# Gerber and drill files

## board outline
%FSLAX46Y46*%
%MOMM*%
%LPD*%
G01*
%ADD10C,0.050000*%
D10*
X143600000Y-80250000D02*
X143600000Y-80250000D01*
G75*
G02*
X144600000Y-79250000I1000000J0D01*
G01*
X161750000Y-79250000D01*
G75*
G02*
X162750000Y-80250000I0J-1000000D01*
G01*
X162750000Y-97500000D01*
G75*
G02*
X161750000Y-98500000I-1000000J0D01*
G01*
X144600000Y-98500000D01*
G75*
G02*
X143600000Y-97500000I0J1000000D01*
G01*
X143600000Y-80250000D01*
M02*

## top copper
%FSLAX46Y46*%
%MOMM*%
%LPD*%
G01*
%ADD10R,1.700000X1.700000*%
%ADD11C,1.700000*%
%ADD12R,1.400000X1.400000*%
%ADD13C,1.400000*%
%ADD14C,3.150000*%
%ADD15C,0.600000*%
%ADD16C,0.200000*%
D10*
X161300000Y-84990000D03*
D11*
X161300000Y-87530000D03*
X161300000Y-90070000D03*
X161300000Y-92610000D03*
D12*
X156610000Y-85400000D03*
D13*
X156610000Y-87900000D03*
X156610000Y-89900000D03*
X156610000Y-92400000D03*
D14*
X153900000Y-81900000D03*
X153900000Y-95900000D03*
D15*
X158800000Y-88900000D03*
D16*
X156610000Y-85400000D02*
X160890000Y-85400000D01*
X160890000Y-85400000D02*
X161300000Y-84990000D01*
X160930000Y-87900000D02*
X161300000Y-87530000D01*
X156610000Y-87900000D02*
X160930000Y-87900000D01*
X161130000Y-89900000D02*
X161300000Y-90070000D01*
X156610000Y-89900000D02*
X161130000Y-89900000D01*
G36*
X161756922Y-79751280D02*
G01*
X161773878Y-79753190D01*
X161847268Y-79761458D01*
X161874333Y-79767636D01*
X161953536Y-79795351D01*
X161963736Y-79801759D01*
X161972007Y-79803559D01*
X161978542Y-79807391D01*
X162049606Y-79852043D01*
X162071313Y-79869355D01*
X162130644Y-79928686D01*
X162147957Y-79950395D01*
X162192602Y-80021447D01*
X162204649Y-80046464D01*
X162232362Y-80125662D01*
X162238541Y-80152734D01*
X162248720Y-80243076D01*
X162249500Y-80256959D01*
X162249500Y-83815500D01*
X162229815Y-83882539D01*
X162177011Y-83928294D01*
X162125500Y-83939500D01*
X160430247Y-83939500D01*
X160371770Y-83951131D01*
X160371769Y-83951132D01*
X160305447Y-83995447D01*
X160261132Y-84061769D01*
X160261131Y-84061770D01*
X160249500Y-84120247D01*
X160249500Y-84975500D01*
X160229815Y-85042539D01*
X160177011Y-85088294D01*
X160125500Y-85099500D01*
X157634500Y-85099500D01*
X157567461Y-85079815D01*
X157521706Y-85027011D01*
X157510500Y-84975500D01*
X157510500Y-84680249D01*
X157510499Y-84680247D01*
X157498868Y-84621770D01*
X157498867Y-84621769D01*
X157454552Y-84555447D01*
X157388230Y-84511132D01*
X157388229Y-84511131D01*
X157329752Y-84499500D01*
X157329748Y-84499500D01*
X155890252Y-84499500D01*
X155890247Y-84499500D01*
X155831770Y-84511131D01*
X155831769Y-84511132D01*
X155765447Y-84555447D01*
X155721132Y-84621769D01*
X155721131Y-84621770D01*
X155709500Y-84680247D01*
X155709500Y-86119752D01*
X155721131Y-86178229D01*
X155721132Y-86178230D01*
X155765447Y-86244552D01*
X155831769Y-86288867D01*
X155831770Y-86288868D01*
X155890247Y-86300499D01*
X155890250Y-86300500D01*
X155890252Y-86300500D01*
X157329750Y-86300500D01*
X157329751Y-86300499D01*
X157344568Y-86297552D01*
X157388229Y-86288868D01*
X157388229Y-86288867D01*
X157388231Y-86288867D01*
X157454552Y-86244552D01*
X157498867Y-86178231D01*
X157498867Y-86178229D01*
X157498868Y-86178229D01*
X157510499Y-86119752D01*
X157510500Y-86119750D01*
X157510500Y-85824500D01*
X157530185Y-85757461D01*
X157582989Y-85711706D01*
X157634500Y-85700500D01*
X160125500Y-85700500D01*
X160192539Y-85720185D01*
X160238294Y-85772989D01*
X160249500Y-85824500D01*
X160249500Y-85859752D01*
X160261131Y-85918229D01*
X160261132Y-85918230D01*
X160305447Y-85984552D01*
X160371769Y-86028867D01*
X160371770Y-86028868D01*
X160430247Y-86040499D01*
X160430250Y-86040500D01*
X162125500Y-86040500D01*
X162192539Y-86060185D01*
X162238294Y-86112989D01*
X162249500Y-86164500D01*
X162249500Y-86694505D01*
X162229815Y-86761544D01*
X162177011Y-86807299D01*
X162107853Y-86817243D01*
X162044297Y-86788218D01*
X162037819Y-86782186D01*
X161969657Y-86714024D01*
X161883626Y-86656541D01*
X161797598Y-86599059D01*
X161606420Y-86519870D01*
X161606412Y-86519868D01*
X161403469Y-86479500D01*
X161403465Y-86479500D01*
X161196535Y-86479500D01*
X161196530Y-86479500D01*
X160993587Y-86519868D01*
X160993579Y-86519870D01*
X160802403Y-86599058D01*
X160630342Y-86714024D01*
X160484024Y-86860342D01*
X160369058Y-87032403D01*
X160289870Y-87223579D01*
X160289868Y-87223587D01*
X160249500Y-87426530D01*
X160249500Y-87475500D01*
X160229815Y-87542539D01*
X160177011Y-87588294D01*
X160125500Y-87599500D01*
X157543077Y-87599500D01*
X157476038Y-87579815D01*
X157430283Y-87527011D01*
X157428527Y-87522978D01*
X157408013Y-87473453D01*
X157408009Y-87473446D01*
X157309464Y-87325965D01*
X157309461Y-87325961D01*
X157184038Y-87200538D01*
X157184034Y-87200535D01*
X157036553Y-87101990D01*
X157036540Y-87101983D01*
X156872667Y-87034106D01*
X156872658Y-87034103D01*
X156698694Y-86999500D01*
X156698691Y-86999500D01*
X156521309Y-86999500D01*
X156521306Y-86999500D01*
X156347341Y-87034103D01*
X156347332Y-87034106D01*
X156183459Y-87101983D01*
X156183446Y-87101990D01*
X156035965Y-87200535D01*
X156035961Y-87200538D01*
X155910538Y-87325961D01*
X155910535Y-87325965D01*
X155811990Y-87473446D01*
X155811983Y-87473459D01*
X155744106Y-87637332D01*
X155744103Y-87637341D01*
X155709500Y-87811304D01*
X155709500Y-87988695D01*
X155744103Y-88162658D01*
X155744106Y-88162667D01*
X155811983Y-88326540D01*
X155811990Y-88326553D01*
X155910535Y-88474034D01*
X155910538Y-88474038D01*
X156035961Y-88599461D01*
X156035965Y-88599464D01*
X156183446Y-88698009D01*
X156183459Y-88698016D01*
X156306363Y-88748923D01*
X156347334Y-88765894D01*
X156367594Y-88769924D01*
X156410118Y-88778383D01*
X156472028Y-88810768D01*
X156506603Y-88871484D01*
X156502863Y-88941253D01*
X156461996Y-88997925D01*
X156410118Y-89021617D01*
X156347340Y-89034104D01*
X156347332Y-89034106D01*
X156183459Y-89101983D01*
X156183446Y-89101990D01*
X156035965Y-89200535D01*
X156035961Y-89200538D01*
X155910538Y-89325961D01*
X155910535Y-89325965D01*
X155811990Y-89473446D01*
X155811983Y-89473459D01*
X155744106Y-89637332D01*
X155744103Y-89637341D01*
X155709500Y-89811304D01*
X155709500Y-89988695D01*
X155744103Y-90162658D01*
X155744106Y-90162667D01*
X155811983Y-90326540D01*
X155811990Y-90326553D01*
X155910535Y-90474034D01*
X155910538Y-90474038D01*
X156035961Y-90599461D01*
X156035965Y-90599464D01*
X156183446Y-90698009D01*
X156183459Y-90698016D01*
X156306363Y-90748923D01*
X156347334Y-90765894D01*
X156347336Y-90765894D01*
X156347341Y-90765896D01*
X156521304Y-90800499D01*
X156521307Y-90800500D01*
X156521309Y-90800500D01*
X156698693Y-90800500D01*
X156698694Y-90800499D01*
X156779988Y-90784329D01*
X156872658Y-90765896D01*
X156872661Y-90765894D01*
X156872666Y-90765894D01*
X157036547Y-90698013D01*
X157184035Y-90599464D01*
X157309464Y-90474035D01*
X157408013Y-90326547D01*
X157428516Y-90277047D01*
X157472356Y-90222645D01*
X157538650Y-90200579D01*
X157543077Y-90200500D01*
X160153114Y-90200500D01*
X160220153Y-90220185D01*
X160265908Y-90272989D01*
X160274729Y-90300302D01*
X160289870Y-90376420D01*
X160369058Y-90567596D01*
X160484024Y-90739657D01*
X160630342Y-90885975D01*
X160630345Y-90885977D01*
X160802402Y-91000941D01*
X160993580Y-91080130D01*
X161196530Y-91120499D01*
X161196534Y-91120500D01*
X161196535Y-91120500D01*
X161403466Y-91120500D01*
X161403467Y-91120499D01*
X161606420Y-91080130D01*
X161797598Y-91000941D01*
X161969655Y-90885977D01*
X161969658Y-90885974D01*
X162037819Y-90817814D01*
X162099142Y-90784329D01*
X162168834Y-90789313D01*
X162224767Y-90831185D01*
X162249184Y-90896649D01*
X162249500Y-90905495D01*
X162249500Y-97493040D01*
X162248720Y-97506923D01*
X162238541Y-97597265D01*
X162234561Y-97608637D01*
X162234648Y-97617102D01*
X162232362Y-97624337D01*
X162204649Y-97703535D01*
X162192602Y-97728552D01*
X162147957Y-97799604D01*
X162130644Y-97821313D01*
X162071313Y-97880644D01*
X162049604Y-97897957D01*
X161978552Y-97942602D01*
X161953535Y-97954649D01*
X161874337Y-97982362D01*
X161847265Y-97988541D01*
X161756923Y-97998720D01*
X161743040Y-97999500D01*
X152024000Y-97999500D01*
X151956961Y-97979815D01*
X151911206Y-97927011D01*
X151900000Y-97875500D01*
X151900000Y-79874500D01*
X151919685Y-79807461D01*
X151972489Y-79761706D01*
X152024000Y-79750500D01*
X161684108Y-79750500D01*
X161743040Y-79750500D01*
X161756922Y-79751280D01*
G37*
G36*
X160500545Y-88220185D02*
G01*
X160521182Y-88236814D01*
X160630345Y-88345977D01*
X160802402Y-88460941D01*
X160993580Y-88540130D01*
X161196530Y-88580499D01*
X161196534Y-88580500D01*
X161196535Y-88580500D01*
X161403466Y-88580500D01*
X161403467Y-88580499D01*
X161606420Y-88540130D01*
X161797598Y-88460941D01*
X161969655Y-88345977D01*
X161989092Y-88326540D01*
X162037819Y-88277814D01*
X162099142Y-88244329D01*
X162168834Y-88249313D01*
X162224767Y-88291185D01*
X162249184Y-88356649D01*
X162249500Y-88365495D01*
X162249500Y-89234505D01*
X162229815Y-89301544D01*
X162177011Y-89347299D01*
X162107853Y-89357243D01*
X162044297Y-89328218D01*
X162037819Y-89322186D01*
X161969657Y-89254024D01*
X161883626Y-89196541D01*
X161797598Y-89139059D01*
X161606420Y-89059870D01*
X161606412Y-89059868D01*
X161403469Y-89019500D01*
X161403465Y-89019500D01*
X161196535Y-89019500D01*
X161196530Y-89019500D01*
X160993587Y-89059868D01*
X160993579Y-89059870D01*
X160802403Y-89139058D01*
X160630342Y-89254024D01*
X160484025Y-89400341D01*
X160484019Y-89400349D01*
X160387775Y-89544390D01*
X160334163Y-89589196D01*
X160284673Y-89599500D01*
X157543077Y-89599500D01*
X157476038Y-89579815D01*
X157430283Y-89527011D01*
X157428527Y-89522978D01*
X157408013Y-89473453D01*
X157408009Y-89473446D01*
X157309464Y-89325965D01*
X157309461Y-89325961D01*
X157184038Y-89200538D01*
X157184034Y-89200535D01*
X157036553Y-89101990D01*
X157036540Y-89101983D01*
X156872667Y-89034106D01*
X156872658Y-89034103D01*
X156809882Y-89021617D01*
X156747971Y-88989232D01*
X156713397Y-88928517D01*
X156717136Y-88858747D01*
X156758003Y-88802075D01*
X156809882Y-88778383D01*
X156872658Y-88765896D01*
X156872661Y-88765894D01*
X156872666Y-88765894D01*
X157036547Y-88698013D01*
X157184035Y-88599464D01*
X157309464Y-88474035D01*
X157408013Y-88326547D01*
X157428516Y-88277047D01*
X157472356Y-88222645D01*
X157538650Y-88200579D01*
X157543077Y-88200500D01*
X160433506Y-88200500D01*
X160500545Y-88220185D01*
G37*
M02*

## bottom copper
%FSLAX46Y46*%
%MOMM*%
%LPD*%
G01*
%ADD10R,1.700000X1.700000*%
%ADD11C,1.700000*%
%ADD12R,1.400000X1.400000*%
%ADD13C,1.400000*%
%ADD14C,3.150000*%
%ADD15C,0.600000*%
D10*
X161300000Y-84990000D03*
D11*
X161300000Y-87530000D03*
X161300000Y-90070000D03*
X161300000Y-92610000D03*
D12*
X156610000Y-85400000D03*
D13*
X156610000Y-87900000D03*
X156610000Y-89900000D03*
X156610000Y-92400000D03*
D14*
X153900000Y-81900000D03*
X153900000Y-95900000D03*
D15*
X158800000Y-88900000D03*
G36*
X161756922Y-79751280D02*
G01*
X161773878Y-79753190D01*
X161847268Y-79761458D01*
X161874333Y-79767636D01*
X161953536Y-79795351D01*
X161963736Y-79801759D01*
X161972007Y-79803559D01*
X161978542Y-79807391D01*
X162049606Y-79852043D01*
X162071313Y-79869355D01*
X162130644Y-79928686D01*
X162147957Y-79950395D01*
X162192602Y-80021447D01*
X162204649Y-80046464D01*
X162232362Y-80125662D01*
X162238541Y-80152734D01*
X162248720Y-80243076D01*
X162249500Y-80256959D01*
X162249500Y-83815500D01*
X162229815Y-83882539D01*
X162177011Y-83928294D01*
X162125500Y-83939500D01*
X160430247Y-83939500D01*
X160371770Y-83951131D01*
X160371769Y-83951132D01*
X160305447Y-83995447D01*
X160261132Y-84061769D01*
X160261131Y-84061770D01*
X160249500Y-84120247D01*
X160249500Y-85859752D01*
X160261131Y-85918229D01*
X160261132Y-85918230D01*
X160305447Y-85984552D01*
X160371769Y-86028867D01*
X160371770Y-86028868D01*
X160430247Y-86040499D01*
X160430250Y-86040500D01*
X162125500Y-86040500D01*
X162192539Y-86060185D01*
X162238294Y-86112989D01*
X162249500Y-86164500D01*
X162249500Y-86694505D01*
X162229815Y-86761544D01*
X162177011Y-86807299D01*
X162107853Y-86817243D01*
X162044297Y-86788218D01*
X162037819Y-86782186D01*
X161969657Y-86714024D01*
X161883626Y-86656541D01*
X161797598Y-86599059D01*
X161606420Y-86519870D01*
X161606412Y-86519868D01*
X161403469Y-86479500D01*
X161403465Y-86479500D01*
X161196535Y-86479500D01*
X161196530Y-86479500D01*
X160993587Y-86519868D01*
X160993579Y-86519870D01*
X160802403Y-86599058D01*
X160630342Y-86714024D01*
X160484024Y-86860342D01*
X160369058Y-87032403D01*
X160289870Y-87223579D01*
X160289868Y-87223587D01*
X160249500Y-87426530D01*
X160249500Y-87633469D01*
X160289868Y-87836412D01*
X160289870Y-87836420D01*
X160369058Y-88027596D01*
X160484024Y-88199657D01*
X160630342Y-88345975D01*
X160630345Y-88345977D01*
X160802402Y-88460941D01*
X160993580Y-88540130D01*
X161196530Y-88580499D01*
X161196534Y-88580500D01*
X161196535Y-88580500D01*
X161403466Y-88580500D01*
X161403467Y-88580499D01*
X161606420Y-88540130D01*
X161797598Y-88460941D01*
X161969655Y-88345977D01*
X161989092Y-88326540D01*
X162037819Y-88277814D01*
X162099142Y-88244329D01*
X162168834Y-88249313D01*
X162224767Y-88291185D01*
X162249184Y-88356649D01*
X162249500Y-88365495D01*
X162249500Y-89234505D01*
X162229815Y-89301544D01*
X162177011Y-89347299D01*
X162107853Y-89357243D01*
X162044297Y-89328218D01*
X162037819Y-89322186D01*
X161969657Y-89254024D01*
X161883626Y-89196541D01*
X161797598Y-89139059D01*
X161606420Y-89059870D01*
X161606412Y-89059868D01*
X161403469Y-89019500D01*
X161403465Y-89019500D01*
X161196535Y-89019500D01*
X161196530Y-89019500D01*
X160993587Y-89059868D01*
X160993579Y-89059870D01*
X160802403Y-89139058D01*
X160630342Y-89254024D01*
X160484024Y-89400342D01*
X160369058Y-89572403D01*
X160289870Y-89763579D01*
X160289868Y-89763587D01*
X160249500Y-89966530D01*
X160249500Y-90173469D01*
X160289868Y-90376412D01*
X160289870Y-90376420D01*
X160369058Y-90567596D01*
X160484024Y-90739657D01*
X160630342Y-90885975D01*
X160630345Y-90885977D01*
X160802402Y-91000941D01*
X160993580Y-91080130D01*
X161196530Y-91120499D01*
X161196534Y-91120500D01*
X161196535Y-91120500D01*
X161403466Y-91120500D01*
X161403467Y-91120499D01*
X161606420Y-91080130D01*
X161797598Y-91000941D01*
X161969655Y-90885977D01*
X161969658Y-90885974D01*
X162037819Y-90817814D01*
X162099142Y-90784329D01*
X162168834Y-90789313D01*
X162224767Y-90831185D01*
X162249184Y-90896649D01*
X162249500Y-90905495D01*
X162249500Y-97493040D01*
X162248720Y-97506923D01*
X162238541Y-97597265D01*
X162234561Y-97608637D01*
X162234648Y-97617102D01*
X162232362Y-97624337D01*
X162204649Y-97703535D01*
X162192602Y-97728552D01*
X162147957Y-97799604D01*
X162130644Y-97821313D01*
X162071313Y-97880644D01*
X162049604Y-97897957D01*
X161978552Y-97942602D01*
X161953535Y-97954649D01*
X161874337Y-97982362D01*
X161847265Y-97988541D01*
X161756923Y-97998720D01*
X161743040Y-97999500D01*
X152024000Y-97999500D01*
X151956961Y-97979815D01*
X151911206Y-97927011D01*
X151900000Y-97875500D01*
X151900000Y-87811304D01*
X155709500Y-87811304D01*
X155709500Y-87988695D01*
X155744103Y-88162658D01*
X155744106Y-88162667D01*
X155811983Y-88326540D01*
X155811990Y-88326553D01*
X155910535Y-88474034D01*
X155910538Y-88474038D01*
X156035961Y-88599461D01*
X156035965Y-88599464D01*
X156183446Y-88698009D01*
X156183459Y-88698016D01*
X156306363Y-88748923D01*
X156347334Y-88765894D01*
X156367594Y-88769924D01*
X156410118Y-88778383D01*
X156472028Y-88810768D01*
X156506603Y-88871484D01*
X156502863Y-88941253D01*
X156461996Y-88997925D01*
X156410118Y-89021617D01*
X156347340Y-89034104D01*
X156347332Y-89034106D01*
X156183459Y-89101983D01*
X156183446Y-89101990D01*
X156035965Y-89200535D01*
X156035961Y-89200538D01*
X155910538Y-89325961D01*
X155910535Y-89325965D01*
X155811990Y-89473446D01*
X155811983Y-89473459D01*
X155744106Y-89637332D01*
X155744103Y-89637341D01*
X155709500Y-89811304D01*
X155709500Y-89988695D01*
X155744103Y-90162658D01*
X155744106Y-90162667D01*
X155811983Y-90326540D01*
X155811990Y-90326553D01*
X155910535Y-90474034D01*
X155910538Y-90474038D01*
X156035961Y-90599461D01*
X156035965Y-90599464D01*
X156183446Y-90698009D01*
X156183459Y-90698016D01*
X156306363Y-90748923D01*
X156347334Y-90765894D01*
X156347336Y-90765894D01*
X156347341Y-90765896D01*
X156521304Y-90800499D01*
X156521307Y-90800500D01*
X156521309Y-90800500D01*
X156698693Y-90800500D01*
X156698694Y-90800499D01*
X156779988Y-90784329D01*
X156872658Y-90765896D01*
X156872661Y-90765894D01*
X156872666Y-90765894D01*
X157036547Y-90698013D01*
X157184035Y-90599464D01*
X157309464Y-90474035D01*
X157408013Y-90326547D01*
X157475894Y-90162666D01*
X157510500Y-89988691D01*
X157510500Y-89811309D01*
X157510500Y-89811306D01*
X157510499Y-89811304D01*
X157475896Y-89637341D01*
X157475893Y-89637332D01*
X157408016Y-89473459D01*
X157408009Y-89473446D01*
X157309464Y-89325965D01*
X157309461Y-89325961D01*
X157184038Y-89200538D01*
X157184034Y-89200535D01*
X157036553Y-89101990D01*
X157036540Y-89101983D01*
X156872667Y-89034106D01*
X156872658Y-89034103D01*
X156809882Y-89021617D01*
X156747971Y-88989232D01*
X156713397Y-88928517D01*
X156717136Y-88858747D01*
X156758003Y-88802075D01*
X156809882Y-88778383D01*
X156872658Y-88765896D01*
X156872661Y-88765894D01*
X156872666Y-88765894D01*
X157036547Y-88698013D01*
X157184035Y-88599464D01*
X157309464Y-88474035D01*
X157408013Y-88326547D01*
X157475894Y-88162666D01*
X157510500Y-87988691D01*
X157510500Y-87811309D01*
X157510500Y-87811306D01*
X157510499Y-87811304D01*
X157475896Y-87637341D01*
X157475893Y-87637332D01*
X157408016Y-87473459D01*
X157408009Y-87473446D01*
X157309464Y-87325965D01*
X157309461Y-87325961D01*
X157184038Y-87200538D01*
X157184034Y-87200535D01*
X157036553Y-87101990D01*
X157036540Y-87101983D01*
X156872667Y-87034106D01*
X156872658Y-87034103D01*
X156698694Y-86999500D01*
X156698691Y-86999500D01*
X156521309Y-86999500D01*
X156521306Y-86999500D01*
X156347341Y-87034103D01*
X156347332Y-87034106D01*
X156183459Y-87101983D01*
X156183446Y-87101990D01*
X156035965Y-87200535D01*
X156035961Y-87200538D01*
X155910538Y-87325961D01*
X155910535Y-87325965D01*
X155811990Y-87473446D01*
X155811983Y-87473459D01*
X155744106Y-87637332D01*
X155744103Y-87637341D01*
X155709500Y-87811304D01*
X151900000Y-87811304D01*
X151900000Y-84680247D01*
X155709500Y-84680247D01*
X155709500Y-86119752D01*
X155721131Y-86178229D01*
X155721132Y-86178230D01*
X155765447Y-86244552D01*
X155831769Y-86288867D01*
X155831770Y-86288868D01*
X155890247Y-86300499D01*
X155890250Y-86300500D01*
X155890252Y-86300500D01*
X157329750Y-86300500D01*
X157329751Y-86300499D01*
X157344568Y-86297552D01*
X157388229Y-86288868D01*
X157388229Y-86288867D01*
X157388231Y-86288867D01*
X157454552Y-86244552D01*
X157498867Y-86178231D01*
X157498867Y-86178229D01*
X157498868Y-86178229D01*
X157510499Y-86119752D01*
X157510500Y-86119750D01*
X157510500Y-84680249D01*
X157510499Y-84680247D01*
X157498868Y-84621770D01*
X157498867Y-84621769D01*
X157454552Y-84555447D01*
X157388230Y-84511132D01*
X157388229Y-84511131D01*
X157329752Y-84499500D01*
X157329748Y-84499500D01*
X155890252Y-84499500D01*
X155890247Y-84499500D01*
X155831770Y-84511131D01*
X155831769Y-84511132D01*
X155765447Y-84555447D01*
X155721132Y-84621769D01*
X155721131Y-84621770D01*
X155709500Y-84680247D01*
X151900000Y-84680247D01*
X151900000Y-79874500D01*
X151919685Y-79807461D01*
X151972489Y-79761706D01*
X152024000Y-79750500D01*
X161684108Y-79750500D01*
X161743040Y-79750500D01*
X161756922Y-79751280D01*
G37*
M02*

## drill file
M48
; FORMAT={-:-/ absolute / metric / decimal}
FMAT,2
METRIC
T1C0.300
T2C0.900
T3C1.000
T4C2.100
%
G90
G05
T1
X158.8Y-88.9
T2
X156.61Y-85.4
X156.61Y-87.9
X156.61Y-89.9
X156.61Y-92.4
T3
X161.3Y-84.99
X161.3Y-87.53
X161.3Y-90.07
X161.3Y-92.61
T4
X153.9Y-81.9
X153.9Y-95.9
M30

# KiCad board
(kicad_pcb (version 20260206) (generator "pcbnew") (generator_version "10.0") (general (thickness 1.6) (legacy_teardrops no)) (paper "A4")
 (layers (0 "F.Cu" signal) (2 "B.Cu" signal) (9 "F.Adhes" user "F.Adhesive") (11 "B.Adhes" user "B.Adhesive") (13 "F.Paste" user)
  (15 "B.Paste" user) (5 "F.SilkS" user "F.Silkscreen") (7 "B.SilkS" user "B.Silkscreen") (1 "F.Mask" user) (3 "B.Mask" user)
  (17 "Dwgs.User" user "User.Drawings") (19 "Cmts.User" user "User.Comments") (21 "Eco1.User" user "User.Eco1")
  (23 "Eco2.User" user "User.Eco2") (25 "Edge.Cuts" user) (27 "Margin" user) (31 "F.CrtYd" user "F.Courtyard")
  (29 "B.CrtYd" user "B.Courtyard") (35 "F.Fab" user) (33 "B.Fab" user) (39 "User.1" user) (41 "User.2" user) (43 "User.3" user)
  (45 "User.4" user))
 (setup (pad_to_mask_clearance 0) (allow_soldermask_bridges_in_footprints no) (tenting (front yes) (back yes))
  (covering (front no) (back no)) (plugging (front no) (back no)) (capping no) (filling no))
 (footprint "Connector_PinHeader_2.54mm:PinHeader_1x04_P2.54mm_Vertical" (layer "F.Cu") (at 161.3 84.99)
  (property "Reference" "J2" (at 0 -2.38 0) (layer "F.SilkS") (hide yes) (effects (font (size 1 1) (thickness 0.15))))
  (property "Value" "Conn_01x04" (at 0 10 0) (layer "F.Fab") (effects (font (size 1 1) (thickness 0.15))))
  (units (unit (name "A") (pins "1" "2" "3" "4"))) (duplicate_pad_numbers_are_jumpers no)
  (pad "1" thru_hole rect (at 0 0) (size 1.7 1.7) (drill 1) (layers "*.Cu" "*.Mask") (remove_unused_layers no) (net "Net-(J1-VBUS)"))
  (pad "2" thru_hole circle (at 0 2.54) (size 1.7 1.7) (drill 1) (layers "*.Cu" "*.Mask") (remove_unused_layers no) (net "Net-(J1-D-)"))
  (pad "3" thru_hole circle (at 0 5.08) (size 1.7 1.7) (drill 1) (layers "*.Cu" "*.Mask") (remove_unused_layers no) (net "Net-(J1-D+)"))
  (pad "4" thru_hole circle (at 0 7.62) (size 1.7 1.7) (drill 1) (layers "*.Cu" "*.Mask") (remove_unused_layers no) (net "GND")))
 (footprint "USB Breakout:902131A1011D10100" (layer "F.Cu") (at 156.61 85.4 -90)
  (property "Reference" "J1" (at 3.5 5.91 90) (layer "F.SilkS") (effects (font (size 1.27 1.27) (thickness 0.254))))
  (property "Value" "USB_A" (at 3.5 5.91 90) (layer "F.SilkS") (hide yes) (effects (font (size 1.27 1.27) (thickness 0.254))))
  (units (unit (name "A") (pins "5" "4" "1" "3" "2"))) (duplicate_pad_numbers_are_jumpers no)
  (pad "1" thru_hole rect (at 0 0 270) (size 1.4 1.4) (drill 0.9) (layers "*.Cu" "*.Mask") (remove_unused_layers no) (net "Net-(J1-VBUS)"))
  (pad "2" thru_hole circle (at 2.5 0 270) (size 1.4 1.4) (drill 0.9) (layers "*.Cu" "*.Mask") (remove_unused_layers no) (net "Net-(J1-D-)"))
  (pad "3" thru_hole circle (at 4.5 0 270) (size 1.4 1.4) (drill 0.9) (layers "*.Cu" "*.Mask") (remove_unused_layers no) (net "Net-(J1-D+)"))
  (pad "4" thru_hole circle (at 7 0 270) (size 1.4 1.4) (drill 0.9) (layers "*.Cu" "*.Mask") (remove_unused_layers no) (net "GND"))
  (pad "5" thru_hole circle (at -3.5 2.71 270) (size 3.15 3.15) (drill 2.1) (layers "*.Cu" "*.Mask") (remove_unused_layers no) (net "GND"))
  (pad "5" thru_hole circle (at 10.5 2.71 270) (size 3.15 3.15) (drill 2.1) (layers "*.Cu" "*.Mask") (remove_unused_layers no) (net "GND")))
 (gr_rect (start 143.6 79.25) (end 162.75 98.5) (radius 1) (stroke (width 0.05) (type solid)) (fill no) (layer "Edge.Cuts"))
 (segment (start 156.61 85.4) (end 160.89 85.4) (width 0.2) (layer "F.Cu") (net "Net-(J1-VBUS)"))
 (segment (start 160.89 85.4) (end 161.3 84.99) (width 0.2) (layer "F.Cu") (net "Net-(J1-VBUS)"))
 (segment (start 160.93 87.9) (end 161.3 87.53) (width 0.2) (layer "F.Cu") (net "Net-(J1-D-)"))
 (segment (start 156.61 87.9) (end 160.93 87.9) (width 0.2) (layer "F.Cu") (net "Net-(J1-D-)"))
 (segment (start 161.13 89.9) (end 161.3 90.07) (width 0.2) (layer "F.Cu") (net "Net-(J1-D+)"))
 (segment (start 156.61 89.9) (end 161.13 89.9) (width 0.2) (layer "F.Cu") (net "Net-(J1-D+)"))
 (via (at 158.8 88.9) (size 0.6) (drill 0.3) (layers "F.Cu" "B.Cu") (free yes) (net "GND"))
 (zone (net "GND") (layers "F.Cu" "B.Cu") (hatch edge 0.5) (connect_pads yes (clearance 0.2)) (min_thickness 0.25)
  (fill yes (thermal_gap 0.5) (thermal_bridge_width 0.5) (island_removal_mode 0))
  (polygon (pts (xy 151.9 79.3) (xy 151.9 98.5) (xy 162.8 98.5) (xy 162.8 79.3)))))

